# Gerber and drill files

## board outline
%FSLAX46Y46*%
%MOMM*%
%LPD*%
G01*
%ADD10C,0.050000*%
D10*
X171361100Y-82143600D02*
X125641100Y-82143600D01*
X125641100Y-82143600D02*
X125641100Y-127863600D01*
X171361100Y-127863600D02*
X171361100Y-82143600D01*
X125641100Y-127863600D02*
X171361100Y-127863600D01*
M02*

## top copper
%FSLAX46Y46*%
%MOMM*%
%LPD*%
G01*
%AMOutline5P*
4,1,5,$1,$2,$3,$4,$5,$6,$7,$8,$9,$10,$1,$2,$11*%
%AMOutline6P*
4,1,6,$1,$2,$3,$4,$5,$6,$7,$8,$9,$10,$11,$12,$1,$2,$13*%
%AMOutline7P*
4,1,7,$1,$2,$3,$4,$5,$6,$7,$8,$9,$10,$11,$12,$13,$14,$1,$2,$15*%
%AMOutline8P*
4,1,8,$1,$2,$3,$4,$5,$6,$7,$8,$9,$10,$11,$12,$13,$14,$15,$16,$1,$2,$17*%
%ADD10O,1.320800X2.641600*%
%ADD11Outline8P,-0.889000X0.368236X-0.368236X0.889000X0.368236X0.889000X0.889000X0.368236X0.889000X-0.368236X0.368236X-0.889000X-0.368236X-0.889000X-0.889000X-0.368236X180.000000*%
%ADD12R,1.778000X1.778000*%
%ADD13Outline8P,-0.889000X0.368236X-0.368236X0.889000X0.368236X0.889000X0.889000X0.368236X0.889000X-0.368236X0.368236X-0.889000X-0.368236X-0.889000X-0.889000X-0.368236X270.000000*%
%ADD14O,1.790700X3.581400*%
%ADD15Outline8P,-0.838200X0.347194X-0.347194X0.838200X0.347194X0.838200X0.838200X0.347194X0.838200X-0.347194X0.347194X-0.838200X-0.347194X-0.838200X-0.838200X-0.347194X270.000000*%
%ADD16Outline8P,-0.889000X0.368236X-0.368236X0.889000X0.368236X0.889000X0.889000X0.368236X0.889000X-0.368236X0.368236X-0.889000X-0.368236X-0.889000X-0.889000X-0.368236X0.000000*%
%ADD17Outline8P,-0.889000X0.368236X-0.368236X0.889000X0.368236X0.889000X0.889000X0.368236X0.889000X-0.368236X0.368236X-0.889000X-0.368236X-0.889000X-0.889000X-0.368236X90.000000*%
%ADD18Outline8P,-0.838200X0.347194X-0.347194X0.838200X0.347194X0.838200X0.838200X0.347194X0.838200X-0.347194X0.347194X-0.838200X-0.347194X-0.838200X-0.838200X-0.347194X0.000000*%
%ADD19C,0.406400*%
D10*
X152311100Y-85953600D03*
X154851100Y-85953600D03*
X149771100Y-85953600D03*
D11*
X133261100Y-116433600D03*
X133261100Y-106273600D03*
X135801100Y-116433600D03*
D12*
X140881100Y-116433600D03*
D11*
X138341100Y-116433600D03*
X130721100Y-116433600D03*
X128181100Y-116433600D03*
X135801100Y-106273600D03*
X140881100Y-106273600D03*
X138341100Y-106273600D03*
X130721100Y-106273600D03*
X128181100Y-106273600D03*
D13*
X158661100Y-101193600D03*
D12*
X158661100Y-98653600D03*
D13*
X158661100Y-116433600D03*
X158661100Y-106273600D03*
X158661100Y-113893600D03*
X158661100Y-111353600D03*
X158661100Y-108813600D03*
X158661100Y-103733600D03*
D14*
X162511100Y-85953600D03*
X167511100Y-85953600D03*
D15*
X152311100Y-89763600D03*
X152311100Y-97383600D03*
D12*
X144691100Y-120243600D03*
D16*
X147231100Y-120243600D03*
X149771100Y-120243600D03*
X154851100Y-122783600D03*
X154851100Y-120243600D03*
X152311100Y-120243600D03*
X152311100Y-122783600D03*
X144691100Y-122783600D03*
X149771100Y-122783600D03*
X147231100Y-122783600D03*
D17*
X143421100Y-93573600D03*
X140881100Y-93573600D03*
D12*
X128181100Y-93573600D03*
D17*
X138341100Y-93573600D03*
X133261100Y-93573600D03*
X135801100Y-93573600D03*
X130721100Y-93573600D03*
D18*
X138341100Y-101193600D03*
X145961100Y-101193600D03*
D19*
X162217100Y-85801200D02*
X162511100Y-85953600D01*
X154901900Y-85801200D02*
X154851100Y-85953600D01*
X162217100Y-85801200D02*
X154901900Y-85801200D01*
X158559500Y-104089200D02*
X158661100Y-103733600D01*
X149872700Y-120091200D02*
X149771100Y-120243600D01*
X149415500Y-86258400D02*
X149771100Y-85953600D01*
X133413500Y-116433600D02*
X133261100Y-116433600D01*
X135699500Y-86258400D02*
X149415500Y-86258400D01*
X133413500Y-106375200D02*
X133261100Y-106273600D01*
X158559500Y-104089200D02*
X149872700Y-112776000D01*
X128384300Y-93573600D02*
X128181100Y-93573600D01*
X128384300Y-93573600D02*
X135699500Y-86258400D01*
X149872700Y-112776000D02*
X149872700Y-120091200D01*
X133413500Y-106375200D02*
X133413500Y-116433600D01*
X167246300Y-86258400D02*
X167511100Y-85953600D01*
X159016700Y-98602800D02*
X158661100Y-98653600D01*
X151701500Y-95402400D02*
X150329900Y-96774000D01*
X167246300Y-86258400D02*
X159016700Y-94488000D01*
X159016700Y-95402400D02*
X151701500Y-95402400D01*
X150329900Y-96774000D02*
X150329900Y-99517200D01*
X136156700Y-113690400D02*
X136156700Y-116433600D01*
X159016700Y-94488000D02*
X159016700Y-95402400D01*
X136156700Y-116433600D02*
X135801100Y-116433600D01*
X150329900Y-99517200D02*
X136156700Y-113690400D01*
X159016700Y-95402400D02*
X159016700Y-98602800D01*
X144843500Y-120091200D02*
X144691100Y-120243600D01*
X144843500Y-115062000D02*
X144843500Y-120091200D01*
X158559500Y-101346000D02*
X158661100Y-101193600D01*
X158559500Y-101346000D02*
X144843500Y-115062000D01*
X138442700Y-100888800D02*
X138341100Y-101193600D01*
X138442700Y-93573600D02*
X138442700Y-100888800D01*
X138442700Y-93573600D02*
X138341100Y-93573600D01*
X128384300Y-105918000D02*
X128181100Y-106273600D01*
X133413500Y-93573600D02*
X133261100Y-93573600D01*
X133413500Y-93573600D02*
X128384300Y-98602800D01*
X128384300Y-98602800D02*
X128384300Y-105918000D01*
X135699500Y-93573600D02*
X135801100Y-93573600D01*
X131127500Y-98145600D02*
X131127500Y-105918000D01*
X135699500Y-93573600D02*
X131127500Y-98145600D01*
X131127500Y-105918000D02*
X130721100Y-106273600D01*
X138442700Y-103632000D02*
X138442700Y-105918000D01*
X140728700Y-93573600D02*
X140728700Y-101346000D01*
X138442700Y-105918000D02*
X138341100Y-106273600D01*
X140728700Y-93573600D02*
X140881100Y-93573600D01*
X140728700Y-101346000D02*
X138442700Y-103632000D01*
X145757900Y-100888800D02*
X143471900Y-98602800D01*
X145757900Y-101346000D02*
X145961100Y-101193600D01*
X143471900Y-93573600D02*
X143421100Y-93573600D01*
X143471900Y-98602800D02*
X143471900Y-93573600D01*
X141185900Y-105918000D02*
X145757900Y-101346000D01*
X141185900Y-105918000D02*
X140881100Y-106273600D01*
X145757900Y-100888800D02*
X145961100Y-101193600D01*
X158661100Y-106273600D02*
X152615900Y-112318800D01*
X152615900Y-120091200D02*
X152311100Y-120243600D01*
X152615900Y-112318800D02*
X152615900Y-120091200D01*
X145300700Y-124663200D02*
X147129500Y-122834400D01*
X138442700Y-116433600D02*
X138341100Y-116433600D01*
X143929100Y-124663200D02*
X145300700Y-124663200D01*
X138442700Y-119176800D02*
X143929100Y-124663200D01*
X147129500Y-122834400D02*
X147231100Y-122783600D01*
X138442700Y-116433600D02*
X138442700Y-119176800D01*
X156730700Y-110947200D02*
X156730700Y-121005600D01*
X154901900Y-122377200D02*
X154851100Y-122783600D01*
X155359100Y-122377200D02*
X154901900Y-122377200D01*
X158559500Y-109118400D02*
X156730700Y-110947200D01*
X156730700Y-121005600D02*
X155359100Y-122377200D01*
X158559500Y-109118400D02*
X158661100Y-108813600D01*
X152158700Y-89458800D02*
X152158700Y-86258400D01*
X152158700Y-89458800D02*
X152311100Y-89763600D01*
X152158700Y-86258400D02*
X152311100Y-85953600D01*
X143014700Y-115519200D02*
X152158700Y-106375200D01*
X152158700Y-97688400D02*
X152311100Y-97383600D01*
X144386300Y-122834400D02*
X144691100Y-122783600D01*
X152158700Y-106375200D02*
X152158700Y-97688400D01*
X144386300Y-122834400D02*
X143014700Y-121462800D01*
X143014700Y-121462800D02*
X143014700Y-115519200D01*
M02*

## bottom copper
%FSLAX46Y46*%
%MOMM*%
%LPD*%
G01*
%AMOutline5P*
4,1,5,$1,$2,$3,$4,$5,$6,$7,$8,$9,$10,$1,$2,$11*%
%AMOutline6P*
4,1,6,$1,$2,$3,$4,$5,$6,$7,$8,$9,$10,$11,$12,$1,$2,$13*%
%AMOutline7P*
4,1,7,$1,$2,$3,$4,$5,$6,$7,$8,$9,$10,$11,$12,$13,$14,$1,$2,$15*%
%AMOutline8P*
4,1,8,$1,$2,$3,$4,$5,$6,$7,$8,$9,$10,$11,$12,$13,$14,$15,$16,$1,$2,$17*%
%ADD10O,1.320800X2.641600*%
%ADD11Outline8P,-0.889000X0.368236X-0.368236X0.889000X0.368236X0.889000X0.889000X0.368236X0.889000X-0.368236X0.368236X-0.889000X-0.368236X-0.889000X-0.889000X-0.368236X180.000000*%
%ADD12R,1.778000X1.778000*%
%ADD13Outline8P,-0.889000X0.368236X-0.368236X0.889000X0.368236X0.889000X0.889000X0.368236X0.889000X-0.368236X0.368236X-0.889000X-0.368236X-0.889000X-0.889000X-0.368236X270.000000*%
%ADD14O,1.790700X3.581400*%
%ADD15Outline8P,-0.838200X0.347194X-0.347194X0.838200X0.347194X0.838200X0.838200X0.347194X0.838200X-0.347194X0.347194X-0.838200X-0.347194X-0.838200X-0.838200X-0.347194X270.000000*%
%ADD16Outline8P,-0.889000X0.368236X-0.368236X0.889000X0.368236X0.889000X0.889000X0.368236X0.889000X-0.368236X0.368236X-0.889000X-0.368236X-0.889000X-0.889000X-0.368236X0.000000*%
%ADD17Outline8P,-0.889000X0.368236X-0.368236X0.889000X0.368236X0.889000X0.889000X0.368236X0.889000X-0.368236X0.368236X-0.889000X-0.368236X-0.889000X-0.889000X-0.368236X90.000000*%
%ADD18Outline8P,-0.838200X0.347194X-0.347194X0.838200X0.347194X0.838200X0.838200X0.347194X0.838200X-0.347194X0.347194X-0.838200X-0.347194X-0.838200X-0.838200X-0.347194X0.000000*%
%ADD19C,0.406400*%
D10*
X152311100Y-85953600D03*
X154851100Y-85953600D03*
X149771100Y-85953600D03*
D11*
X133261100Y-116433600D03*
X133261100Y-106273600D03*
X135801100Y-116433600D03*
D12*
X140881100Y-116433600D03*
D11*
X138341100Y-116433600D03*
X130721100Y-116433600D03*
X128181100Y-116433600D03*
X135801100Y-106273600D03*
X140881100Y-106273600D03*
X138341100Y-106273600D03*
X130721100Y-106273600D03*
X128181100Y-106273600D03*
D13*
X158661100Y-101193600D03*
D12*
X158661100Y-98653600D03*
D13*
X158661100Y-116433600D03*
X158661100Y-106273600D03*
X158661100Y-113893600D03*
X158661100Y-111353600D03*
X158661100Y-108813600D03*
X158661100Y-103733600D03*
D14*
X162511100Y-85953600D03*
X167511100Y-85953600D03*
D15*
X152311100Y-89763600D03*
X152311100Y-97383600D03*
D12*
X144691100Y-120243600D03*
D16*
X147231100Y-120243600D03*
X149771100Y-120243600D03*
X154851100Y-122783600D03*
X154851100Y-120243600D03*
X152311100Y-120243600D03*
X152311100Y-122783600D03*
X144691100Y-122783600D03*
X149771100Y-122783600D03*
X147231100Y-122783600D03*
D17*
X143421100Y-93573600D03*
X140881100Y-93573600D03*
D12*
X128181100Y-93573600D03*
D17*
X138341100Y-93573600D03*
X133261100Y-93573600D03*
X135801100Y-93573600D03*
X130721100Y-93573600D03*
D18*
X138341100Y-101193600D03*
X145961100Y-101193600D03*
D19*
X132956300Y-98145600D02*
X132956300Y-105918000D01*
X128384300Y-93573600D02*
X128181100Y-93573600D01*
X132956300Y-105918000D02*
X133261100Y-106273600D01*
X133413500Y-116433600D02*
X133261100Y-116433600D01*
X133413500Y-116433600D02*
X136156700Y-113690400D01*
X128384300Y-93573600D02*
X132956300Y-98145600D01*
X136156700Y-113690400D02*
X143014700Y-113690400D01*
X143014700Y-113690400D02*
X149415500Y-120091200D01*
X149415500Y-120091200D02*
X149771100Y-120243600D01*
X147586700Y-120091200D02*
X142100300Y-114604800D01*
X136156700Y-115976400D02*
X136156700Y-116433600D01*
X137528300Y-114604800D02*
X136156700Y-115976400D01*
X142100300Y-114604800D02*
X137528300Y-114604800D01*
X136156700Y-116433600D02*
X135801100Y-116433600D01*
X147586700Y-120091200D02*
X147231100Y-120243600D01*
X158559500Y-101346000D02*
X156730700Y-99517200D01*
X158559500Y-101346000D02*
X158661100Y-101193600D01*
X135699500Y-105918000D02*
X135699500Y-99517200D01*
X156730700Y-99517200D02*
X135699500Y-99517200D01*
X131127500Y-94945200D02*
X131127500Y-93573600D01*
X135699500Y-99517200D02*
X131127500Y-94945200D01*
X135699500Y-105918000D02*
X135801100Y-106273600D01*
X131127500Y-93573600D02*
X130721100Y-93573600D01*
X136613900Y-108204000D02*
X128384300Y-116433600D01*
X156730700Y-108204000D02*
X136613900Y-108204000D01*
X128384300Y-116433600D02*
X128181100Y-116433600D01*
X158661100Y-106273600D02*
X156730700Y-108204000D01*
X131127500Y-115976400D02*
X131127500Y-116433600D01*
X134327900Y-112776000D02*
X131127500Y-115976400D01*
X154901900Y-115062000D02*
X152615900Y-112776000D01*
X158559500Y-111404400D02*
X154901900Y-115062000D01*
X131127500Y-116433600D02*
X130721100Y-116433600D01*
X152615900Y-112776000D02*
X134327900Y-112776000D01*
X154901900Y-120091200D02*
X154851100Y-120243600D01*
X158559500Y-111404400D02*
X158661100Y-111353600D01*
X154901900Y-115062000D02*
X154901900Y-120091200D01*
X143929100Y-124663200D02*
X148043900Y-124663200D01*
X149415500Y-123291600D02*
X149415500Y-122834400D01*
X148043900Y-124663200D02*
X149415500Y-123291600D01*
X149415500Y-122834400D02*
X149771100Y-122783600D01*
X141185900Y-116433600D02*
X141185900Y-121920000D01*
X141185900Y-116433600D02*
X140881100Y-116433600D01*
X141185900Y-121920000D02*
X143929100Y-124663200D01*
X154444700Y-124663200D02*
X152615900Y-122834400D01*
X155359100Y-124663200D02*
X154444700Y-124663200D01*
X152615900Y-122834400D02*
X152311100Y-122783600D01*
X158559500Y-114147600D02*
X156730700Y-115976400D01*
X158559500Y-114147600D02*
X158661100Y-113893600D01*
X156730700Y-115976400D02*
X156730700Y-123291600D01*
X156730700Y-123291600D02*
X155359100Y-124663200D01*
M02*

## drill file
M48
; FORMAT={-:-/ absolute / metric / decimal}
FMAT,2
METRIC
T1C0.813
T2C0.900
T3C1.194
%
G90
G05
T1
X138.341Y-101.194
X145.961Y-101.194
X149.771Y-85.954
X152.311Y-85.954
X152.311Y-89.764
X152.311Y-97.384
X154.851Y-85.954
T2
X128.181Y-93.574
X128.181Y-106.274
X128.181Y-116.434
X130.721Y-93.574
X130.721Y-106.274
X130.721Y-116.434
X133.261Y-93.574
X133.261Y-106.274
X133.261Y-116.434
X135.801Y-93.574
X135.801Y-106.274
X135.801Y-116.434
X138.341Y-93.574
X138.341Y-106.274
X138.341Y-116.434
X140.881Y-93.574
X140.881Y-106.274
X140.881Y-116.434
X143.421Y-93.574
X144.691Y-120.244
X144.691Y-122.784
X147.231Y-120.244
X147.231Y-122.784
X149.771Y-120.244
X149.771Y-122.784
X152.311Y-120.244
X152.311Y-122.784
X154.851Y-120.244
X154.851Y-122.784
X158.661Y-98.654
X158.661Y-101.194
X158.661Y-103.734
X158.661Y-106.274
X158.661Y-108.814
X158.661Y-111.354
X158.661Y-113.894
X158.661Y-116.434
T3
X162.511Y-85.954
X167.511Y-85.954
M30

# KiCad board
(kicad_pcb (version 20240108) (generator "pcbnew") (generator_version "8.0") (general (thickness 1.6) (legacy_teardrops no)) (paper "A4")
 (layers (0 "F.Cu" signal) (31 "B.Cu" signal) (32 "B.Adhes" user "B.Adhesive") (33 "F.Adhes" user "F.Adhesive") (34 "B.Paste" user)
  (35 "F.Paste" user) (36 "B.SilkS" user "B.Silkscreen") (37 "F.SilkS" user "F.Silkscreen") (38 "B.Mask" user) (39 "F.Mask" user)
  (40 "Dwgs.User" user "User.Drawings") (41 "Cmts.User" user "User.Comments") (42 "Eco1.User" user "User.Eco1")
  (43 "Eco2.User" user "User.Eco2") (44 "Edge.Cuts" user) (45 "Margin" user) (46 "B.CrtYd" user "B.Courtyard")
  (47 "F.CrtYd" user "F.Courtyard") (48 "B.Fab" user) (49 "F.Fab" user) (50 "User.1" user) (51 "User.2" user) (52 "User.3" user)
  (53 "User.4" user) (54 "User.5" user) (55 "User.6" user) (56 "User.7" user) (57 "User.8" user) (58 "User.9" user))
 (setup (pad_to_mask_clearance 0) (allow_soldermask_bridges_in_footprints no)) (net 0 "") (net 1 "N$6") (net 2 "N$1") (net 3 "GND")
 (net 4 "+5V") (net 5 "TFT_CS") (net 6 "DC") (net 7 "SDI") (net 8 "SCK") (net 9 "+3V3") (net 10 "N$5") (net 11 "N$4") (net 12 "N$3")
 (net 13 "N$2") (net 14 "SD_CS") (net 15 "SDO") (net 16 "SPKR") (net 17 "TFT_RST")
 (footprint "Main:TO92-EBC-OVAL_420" (layer "F.Cu") (at 152.3111 84.6836)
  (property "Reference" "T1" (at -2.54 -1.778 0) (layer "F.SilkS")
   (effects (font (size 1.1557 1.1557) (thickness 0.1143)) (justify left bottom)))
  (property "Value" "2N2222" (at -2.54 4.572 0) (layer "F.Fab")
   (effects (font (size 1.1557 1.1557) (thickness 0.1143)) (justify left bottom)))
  (pad "B" thru_hole oval (at 0 1.27 90) (size 2.6416 1.3208) (drill 0.8128) (layers "*.Cu" "*.Mask") (remove_unused_layers no)
   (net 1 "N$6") (solder_mask_margin 0.1016) (thermal_bridge_angle 0))
  (pad "C" thru_hole oval (at 2.54 1.27 90) (size 2.6416 1.3208) (drill 0.8128) (layers "*.Cu" "*.Mask") (remove_unused_layers no)
   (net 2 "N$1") (solder_mask_margin 0.1016) (thermal_bridge_angle 0))
  (pad "E" thru_hole oval (at -2.54 1.27 90) (size 2.6416 1.3208) (drill 0.8128) (layers "*.Cu" "*.Mask") (remove_unused_layers no)
   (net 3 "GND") (solder_mask_margin 0.1016) (thermal_bridge_angle 0)))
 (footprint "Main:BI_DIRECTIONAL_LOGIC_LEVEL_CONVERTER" (layer "F.Cu") (at 134.5311 111.3536 180)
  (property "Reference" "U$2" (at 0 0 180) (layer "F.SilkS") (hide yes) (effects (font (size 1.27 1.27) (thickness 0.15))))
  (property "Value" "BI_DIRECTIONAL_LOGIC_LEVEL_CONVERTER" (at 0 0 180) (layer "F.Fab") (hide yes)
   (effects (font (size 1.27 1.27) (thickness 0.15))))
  (pad "GND1" thru_hole roundrect (at 1.27 -5.08 180) (size 1.778 1.778) (drill 0.9) (layers "*.Cu" "*.Mask") (remove_unused_layers no)
   (roundrect_rratio 0.25) (chamfer_ratio 0.2928932188) (chamfer top_left top_right bottom_left bottom_right) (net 3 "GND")
   (solder_mask_margin 0.1016) (thermal_bridge_angle 0))
  (pad "GND2" thru_hole roundrect (at 1.27 5.08 180) (size 1.778 1.778) (drill 0.9) (layers "*.Cu" "*.Mask") (remove_unused_layers no)
   (roundrect_rratio 0.25) (chamfer_ratio 0.2928932188) (chamfer top_left top_right bottom_left bottom_right) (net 3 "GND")
   (solder_mask_margin 0.1016) (thermal_bridge_angle 0))
  (pad "HV" thru_hole roundrect (at -1.27 -5.08 180) (size 1.778 1.778) (drill 0.9) (layers "*.Cu" "*.Mask") (remove_unused_layers no)
   (roundrect_rratio 0.25) (chamfer_ratio 0.2928932188) (chamfer top_left top_right bottom_left bottom_right) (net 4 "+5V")
   (solder_mask_margin 0.1016) (thermal_bridge_angle 0))
  (pad "HV1" thru_hole rect (at -6.35 -5.08 180) (size 1.778 1.778) (drill 0.9) (layers "*.Cu" "*.Mask") (remove_unused_layers no)
   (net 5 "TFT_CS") (solder_mask_margin 0.1016) (thermal_bridge_angle 0))
  (pad "HV2" thru_hole roundrect (at -3.81 -5.08 180) (size 1.778 1.778) (drill 0.9) (layers "*.Cu" "*.Mask") (remove_unused_layers no)
   (roundrect_rratio 0.25) (chamfer_ratio 0.2928932188) (chamfer top_left top_right bottom_left bottom_right) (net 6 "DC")
   (solder_mask_margin 0.1016) (thermal_bridge_angle 0))
  (pad "HV3" thru_hole roundrect (at 3.81 -5.08 180) (size 1.778 1.778) (drill 0.9) (layers "*.Cu" "*.Mask") (remove_unused_layers no)
   (roundrect_rratio 0.25) (chamfer_ratio 0.2928932188) (chamfer top_left top_right bottom_left bottom_right) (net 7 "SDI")
   (solder_mask_margin 0.1016) (thermal_bridge_angle 0))
  (pad "HV4" thru_hole roundrect (at 6.35 -5.08 180) (size 1.778 1.778) (drill 0.9) (layers "*.Cu" "*.Mask") (remove_unused_layers no)
   (roundrect_rratio 0.25) (chamfer_ratio 0.2928932188) (chamfer top_left top_right bottom_left bottom_right) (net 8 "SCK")
   (solder_mask_margin 0.1016) (thermal_bridge_angle 0))
  (pad "LV" thru_hole roundrect (at -1.27 5.08 180) (size 1.778 1.778) (drill 0.9) (layers "*.Cu" "*.Mask") (remove_unused_layers no)
   (roundrect_rratio 0.25) (chamfer_ratio 0.2928932188) (chamfer top_left top_right bottom_left bottom_right) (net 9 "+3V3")
   (solder_mask_margin 0.1016) (thermal_bridge_angle 0))
  (pad "LV1" thru_hole roundrect (at -6.35 5.08 180) (size 1.778 1.778) (drill 0.9) (layers "*.Cu" "*.Mask") (remove_unused_layers no)
   (roundrect_rratio 0.25) (chamfer_ratio 0.2928932188) (chamfer top_left top_right bottom_left bottom_right) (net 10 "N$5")
   (solder_mask_margin 0.1016) (thermal_bridge_angle 0))
  (pad "LV2" thru_hole roundrect (at -3.81 5.08 180) (size 1.778 1.778) (drill 0.9) (layers "*.Cu" "*.Mask") (remove_unused_layers no)
   (roundrect_rratio 0.25) (chamfer_ratio 0.2928932188) (chamfer top_left top_right bottom_left bottom_right) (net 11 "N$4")
   (solder_mask_margin 0.1016) (thermal_bridge_angle 0))
  (pad "LV3" thru_hole roundrect (at 3.81 5.08 180) (size 1.778 1.778) (drill 0.9) (layers "*.Cu" "*.Mask") (remove_unused_layers no)
   (roundrect_rratio 0.25) (chamfer_ratio 0.2928932188) (chamfer top_left top_right bottom_left bottom_right) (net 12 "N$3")
   (solder_mask_margin 0.1016) (thermal_bridge_angle 0))
  (pad "LV4" thru_hole roundrect (at 6.35 5.08 180) (size 1.778 1.778) (drill 0.9) (layers "*.Cu" "*.Mask") (remove_unused_layers no)
   (roundrect_rratio 0.25) (chamfer_ratio 0.2928932188) (chamfer top_left top_right bottom_left bottom_right) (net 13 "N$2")
   (solder_mask_margin 0.1016) (thermal_bridge_angle 0)))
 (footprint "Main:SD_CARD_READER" (layer "F.Cu") (at 158.6611 107.5436 -90)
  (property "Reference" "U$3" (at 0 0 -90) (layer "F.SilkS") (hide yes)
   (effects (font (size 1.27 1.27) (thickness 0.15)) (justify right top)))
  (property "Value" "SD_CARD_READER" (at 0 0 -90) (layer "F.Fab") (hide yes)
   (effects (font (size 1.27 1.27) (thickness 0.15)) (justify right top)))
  (pad "3V" thru_hole roundrect (at -6.35 0 270) (size 1.778 1.778) (drill 0.9) (layers "*.Cu" "*.Mask") (remove_unused_layers no)
   (roundrect_rratio 0.25) (chamfer_ratio 0.2928932188) (chamfer top_left top_right bottom_left bottom_right) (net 9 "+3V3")
   (solder_mask_margin 0.1016) (thermal_bridge_angle 0))
  (pad "5V" thru_hole rect (at -8.89 0 270) (size 1.778 1.778) (drill 0.9) (layers "*.Cu" "*.Mask") (remove_unused_layers no) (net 4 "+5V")
   (solder_mask_margin 0.1016) (thermal_bridge_angle 0))
  (pad "CD" thru_hole roundrect (at 8.89 0 270) (size 1.778 1.778) (drill 0.9) (layers "*.Cu" "*.Mask") (remove_unused_layers no)
   (roundrect_rratio 0.25) (chamfer_ratio 0.2928932188) (chamfer top_left top_right bottom_left bottom_right) (solder_mask_margin 0.1016)
   (thermal_bridge_angle 0))
  (pad "CLK" thru_hole roundrect (at -1.27 0 270) (size 1.778 1.778) (drill 0.9) (layers "*.Cu" "*.Mask") (remove_unused_layers no)
   (roundrect_rratio 0.25) (chamfer_ratio 0.2928932188) (chamfer top_left top_right bottom_left bottom_right) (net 8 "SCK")
   (solder_mask_margin 0.1016) (thermal_bridge_angle 0))
  (pad "CS" thru_hole roundrect (at 6.35 0 270) (size 1.778 1.778) (drill 0.9) (layers "*.Cu" "*.Mask") (remove_unused_layers no)
   (roundrect_rratio 0.25) (chamfer_ratio 0.2928932188) (chamfer top_left top_right bottom_left bottom_right) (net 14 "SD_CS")
   (solder_mask_margin 0.1016) (thermal_bridge_angle 0))
  (pad "DI" thru_hole roundrect (at 3.81 0 270) (size 1.778 1.778) (drill 0.9) (layers "*.Cu" "*.Mask") (remove_unused_layers no)
   (roundrect_rratio 0.25) (chamfer_ratio 0.2928932188) (chamfer top_left top_right bottom_left bottom_right) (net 7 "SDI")
   (solder_mask_margin 0.1016) (thermal_bridge_angle 0))
  (pad "DO" thru_hole roundrect (at 1.27 0 270) (size 1.778 1.778) (drill 0.9) (layers "*.Cu" "*.Mask") (remove_unused_layers no)
   (roundrect_rratio 0.25) (chamfer_ratio 0.2928932188) (chamfer top_left top_right bottom_left bottom_right) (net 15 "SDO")
   (solder_mask_margin 0.1016) (thermal_bridge_angle 0))
  (pad "GND" thru_hole roundrect (at -3.81 0 270) (size 1.778 1.778) (drill 0.9) (layers "*.Cu" "*.Mask") (remove_unused_layers no)
   (roundrect_rratio 0.25) (chamfer_ratio 0.2928932188) (chamfer top_left top_right bottom_left bottom_right) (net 3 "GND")
   (solder_mask_margin 0.1016) (thermal_bridge_angle 0)))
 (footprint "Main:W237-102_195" (layer "F.Cu") (at 165.0111 84.6836)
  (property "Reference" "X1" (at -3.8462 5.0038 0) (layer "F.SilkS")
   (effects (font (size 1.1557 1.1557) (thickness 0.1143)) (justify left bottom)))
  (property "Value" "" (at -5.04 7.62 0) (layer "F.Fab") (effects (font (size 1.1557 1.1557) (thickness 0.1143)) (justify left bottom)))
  (pad "1" thru_hole oval (at -2.5 1.27 90) (size 3.5814 1.7907) (drill 1.1938) (layers "*.Cu" "*.Mask") (remove_unused_layers no)
   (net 2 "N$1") (solder_mask_margin 0.1016) (thermal_bridge_angle 0))
  (pad "2" thru_hole oval (at 2.5 1.27 90) (size 3.5814 1.7907) (drill 1.1938) (layers "*.Cu" "*.Mask") (remove_unused_layers no)
   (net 4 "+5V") (solder_mask_margin 0.1016) (thermal_bridge_angle 0)))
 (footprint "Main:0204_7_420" (layer "F.Cu") (at 152.3111 93.5736 -90)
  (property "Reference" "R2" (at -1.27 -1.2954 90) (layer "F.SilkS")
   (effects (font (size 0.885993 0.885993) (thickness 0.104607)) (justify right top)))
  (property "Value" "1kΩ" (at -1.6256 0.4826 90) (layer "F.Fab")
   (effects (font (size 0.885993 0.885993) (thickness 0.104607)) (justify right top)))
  (pad "1" thru_hole roundrect (at -3.81 0 270) (size 1.6764 1.6764) (drill 0.8128) (layers "*.Cu" "*.Mask") (remove_unused_layers no)
   (roundrect_rratio 0.25) (chamfer_ratio 0.2928932188) (chamfer top_left top_right bottom_left bottom_right) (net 1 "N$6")
   (solder_mask_margin 0.1016) (thermal_bridge_angle 0))
  (pad "2" thru_hole roundrect (at 3.81 0 270) (size 1.6764 1.6764) (drill 0.8128) (layers "*.Cu" "*.Mask") (remove_unused_layers no)
   (roundrect_rratio 0.25) (chamfer_ratio 0.2928932188) (chamfer top_left top_right bottom_left bottom_right) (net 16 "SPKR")
   (solder_mask_margin 0.1016) (thermal_bridge_angle 0)))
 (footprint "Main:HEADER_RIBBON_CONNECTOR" (layer "F.Cu") (at 149.7711 121.5136)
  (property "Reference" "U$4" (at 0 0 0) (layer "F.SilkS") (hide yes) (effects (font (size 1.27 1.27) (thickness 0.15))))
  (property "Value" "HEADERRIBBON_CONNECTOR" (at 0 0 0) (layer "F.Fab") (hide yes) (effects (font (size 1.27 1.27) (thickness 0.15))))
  (pad "3V3" thru_hole rect (at -5.08 -1.27) (size 1.778 1.778) (drill 0.9) (layers "*.Cu" "*.Mask") (remove_unused_layers no)
   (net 9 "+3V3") (solder_mask_margin 0.1016) (thermal_bridge_angle 0))
  (pad "5V" thru_hole roundrect (at -2.54 -1.27) (size 1.778 1.778) (drill 0.9) (layers "*.Cu" "*.Mask") (remove_unused_layers no)
   (roundrect_rratio 0.25) (chamfer_ratio 0.2928932188) (chamfer top_left top_right bottom_left bottom_right) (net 4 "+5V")
   (solder_mask_margin 0.1016) (thermal_bridge_angle 0))
  (pad "GND" thru_hole roundrect (at 0 -1.27) (size 1.778 1.778) (drill 0.9) (layers "*.Cu" "*.Mask") (remove_unused_layers no)
   (roundrect_rratio 0.25) (chamfer_ratio 0.2928932188) (chamfer top_left top_right bottom_left bottom_right) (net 3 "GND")
   (solder_mask_margin 0.1016) (thermal_bridge_angle 0))
  (pad "MISO" thru_hole roundrect (at 5.08 1.27) (size 1.778 1.778) (drill 0.9) (layers "*.Cu" "*.Mask") (remove_unused_layers no)
   (roundrect_rratio 0.25) (chamfer_ratio 0.2928932188) (chamfer top_left top_right bottom_left bottom_right) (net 15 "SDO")
   (solder_mask_margin 0.1016) (thermal_bridge_angle 0))
  (pad "MOSI" thru_hole roundrect (at 5.08 -1.27) (size 1.778 1.778) (drill 0.9) (layers "*.Cu" "*.Mask") (remove_unused_layers no)
   (roundrect_rratio 0.25) (chamfer_ratio 0.2928932188) (chamfer top_left top_right bottom_left bottom_right) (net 7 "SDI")
   (solder_mask_margin 0.1016) (thermal_bridge_angle 0))
  (pad "SCK" thru_hole roundrect (at 2.54 -1.27) (size 1.778 1.778) (drill 0.9) (layers "*.Cu" "*.Mask") (remove_unused_layers no)
   (roundrect_rratio 0.25) (chamfer_ratio 0.2928932188) (chamfer top_left top_right bottom_left bottom_right) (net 8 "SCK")
   (solder_mask_margin 0.1016) (thermal_bridge_angle 0))
  (pad "SD_CS" thru_hole roundrect (at 2.54 1.27) (size 1.778 1.778) (drill 0.9) (layers "*.Cu" "*.Mask") (remove_unused_layers no)
   (roundrect_rratio 0.25) (chamfer_ratio 0.2928932188) (chamfer top_left top_right bottom_left bottom_right) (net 14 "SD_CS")
   (solder_mask_margin 0.1016) (thermal_bridge_angle 0))
  (pad "SPKR" thru_hole roundrect (at -5.08 1.27) (size 1.778 1.778) (drill 0.9) (layers "*.Cu" "*.Mask") (remove_unused_layers no)
   (roundrect_rratio 0.25) (chamfer_ratio 0.2928932188) (chamfer top_left top_right bottom_left bottom_right) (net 16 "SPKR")
   (solder_mask_margin 0.1016) (thermal_bridge_angle 0))
  (pad "TFT_CS" thru_hole roundrect (at 0 1.27) (size 1.778 1.778) (drill 0.9) (layers "*.Cu" "*.Mask") (remove_unused_layers no)
   (roundrect_rratio 0.25) (chamfer_ratio 0.2928932188) (chamfer top_left top_right bottom_left bottom_right) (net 5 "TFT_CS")
   (solder_mask_margin 0.1016) (thermal_bridge_angle 0))
  (pad "TFT_DC" thru_hole roundrect (at -2.54 1.27) (size 1.778 1.778) (drill 0.9) (layers "*.Cu" "*.Mask") (remove_unused_layers no)
   (roundrect_rratio 0.25) (chamfer_ratio 0.2928932188) (chamfer top_left top_right bottom_left bottom_right) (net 6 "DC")
   (solder_mask_margin 0.1016) (thermal_bridge_angle 0)))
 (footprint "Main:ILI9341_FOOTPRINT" (layer "F.Cu") (at 135.8011 78.3336 90)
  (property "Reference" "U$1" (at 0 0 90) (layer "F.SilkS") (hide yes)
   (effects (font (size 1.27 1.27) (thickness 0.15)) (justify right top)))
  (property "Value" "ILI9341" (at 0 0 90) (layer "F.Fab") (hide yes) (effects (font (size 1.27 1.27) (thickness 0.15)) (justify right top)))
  (pad "CS" thru_hole roundrect (at -15.24 7.62 90) (size 1.778 1.778) (drill 0.9) (layers "*.Cu" "*.Mask") (remove_unused_layers no)
   (roundrect_rratio 0.25) (chamfer_ratio 0.2928932188) (chamfer top_left top_right bottom_left bottom_right) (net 10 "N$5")
   (solder_mask_margin 0.1016) (thermal_bridge_angle 0))
  (pad "DC" thru_hole roundrect (at -15.24 5.08 90) (size 1.778 1.778) (drill 0.9) (layers "*.Cu" "*.Mask") (remove_unused_layers no)
   (roundrect_rratio 0.25) (chamfer_ratio 0.2928932188) (chamfer top_left top_right bottom_left bottom_right) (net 11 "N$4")
   (solder_mask_margin 0.1016) (thermal_bridge_angle 0))
  (pad "GND" thru_hole rect (at -15.24 -7.62 90) (size 1.778 1.778) (drill 0.9) (layers "*.Cu" "*.Mask") (remove_unused_layers no)
   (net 3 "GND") (solder_mask_margin 0.1016) (thermal_bridge_angle 0))
  (pad "RST" thru_hole roundrect (at -15.24 2.54 90) (size 1.778 1.778) (drill 0.9) (layers "*.Cu" "*.Mask") (remove_unused_layers no)
   (roundrect_rratio 0.25) (chamfer_ratio 0.2928932188) (chamfer top_left top_right bottom_left bottom_right) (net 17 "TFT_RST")
   (solder_mask_margin 0.1016) (thermal_bridge_angle 0))
  (pad "SCK" thru_hole roundrect (at -15.24 -2.54 90) (size 1.778 1.778) (drill 0.9) (layers "*.Cu" "*.Mask") (remove_unused_layers no)
   (roundrect_rratio 0.25) (chamfer_ratio 0.2928932188) (chamfer top_left top_right bottom_left bottom_right) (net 13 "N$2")
   (solder_mask_margin 0.1016) (thermal_bridge_angle 0))
  (pad "SDA" thru_hole roundrect (at -15.24 0 90) (size 1.778 1.778) (drill 0.9) (layers "*.Cu" "*.Mask") (remove_unused_layers no)
   (roundrect_rratio 0.25) (chamfer_ratio 0.2928932188) (chamfer top_left top_right bottom_left bottom_right) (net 12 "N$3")
   (solder_mask_margin 0.1016) (thermal_bridge_angle 0))
  (pad "VCC" thru_hole roundrect (at -15.24 -5.08 90) (size 1.778 1.778) (drill 0.9) (layers "*.Cu" "*.Mask") (remove_unused_layers no)
   (roundrect_rratio 0.25) (chamfer_ratio 0.2928932188) (chamfer top_left top_right bottom_left bottom_right) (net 9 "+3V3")
   (solder_mask_margin 0.1016) (thermal_bridge_angle 0)))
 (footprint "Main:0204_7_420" (layer "F.Cu") (at 142.1511 101.1936)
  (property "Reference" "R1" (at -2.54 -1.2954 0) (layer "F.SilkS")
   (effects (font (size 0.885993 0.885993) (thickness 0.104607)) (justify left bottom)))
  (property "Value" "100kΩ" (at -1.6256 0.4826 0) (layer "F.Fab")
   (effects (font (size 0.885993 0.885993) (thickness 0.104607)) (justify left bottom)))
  (pad "1" thru_hole roundrect (at -3.81 0) (size 1.6764 1.6764) (drill 0.8128) (layers "*.Cu" "*.Mask") (remove_unused_layers no)
   (roundrect_rratio 0.25) (chamfer_ratio 0.2928932188) (chamfer top_left top_right bottom_left bottom_right) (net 17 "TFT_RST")
   (solder_mask_margin 0.1016) (thermal_bridge_angle 0))
  (pad "2" thru_hole roundrect (at 3.81 0) (size 1.6764 1.6764) (drill 0.8128) (layers "*.Cu" "*.Mask") (remove_unused_layers no)
   (roundrect_rratio 0.25) (chamfer_ratio 0.2928932188) (chamfer top_left top_right bottom_left bottom_right) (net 10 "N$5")
   (solder_mask_margin 0.1016) (thermal_bridge_angle 0)))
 (gr_line (start 171.3611 82.1436) (end 125.6411 82.1436) (stroke (width 0.05) (type solid)) (layer "Edge.Cuts"))
 (gr_line (start 125.6411 82.1436) (end 125.6411 127.8636) (stroke (width 0.05) (type solid)) (layer "Edge.Cuts"))
 (gr_line (start 171.3611 127.8636) (end 171.3611 82.1436) (stroke (width 0.05) (type solid)) (layer "Edge.Cuts"))
 (gr_line (start 125.6411 127.8636) (end 171.3611 127.8636) (stroke (width 0.05) (type solid)) (layer "Edge.Cuts"))
 (segment (start 162.2171 85.8012) (end 162.5111 85.9536) (width 0.4064) (layer "F.Cu") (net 2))
 (segment (start 154.9019 85.8012) (end 154.8511 85.9536) (width 0.4064) (layer "F.Cu") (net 2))
 (segment (start 162.2171 85.8012) (end 154.9019 85.8012) (width 0.4064) (layer "F.Cu") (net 2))
 (segment (start 158.5595 104.0892) (end 158.6611 103.7336) (width 0.4064) (layer "F.Cu") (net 3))
 (segment (start 149.8727 120.0912) (end 149.7711 120.2436) (width 0.4064) (layer "F.Cu") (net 3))
 (segment (start 149.4155 86.2584) (end 149.7711 85.9536) (width 0.4064) (layer "F.Cu") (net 3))
 (segment (start 133.4135 116.4336) (end 133.2611 116.4336) (width 0.4064) (layer "F.Cu") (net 3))
 (segment (start 135.6995 86.2584) (end 149.4155 86.2584) (width 0.4064) (layer "F.Cu") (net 3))
 (segment (start 133.4135 106.3752) (end 133.2611 106.2736) (width 0.4064) (layer "F.Cu") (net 3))
 (segment (start 158.5595 104.0892) (end 149.8727 112.776) (width 0.4064) (layer "F.Cu") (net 3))
 (segment (start 128.3843 93.5736) (end 128.1811 93.5736) (width 0.4064) (layer "F.Cu") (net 3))
 (segment (start 128.3843 93.5736) (end 135.6995 86.2584) (width 0.4064) (layer "F.Cu") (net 3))
 (segment (start 149.8727 112.776) (end 149.8727 120.0912) (width 0.4064) (layer "F.Cu") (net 3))
 (segment (start 133.4135 106.3752) (end 133.4135 116.4336) (width 0.4064) (layer "F.Cu") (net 3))
 (segment (start 132.9563 98.1456) (end 132.9563 105.918) (width 0.4064) (layer "B.Cu") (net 3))
 (segment (start 128.3843 93.5736) (end 128.1811 93.5736) (width 0.4064) (layer "B.Cu") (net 3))
 (segment (start 132.9563 105.918) (end 133.2611 106.2736) (width 0.4064) (layer "B.Cu") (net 3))
 (segment (start 133.4135 116.4336) (end 133.2611 116.4336) (width 0.4064) (layer "B.Cu") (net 3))
 (segment (start 133.4135 116.4336) (end 136.1567 113.6904) (width 0.4064) (layer "B.Cu") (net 3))
 (segment (start 128.3843 93.5736) (end 132.9563 98.1456) (width 0.4064) (layer "B.Cu") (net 3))
 (segment (start 136.1567 113.6904) (end 143.0147 113.6904) (width 0.4064) (layer "B.Cu") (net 3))
 (segment (start 143.0147 113.6904) (end 149.4155 120.0912) (width 0.4064) (layer "B.Cu") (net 3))
 (segment (start 149.4155 120.0912) (end 149.7711 120.2436) (width 0.4064) (layer "B.Cu") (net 3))
 (segment (start 167.2463 86.2584) (end 167.5111 85.9536) (width 0.4064) (layer "F.Cu") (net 4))
 (segment (start 159.0167 98.6028) (end 158.6611 98.6536) (width 0.4064) (layer "F.Cu") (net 4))
 (segment (start 151.7015 95.4024) (end 150.3299 96.774) (width 0.4064) (layer "F.Cu") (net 4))
 (segment (start 167.2463 86.2584) (end 159.0167 94.488) (width 0.4064) (layer "F.Cu") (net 4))
 (segment (start 159.0167 95.4024) (end 151.7015 95.4024) (width 0.4064) (layer "F.Cu") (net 4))
 (segment (start 150.3299 96.774) (end 150.3299 99.5172) (width 0.4064) (layer "F.Cu") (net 4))
 (segment (start 136.1567 113.6904) (end 136.1567 116.4336) (width 0.4064) (layer "F.Cu") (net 4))
 (segment (start 159.0167 94.488) (end 159.0167 95.4024) (width 0.4064) (layer "F.Cu") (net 4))
 (segment (start 136.1567 116.4336) (end 135.8011 116.4336) (width 0.4064) (layer "F.Cu") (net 4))
 (segment (start 150.3299 99.5172) (end 136.1567 113.6904) (width 0.4064) (layer "F.Cu") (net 4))
 (segment (start 159.0167 95.4024) (end 159.0167 98.6028) (width 0.4064) (layer "F.Cu") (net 4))
 (segment (start 147.5867 120.0912) (end 142.1003 114.6048) (width 0.4064) (layer "B.Cu") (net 4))
 (segment (start 136.1567 115.9764) (end 136.1567 116.4336) (width 0.4064) (layer "B.Cu") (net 4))
 (segment (start 137.5283 114.6048) (end 136.1567 115.9764) (width 0.4064) (layer "B.Cu") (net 4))
 (segment (start 142.1003 114.6048) (end 137.5283 114.6048) (width 0.4064) (layer "B.Cu") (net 4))
 (segment (start 136.1567 116.4336) (end 135.8011 116.4336) (width 0.4064) (layer "B.Cu") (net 4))
 (segment (start 147.5867 120.0912) (end 147.2311 120.2436) (width 0.4064) (layer "B.Cu") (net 4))
 (segment (start 144.8435 120.0912) (end 144.6911 120.2436) (width 0.4064) (layer "F.Cu") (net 9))
 (segment (start 144.8435 115.062) (end 144.8435 120.0912) (width 0.4064) (layer "F.Cu") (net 9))
 (segment (start 158.5595 101.346) (end 158.6611 101.1936) (width 0.4064) (layer "F.Cu") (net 9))
 (segment (start 158.5595 101.346) (end 144.8435 115.062) (width 0.4064) (layer "F.Cu") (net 9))
 (segment (start 158.5595 101.346) (end 156.7307 99.5172) (width 0.4064) (layer "B.Cu") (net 9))
 (segment (start 158.5595 101.346) (end 158.6611 101.1936) (width 0.4064) (layer "B.Cu") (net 9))
 (segment (start 135.6995 105.918) (end 135.6995 99.5172) (width 0.4064) (layer "B.Cu") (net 9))
 (segment (start 156.7307 99.5172) (end 135.6995 99.5172) (width 0.4064) (layer "B.Cu") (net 9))
 (segment (start 131.1275 94.9452) (end 131.1275 93.5736) (width 0.4064) (layer "B.Cu") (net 9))
 (segment (start 135.6995 99.5172) (end 131.1275 94.9452) (width 0.4064) (layer "B.Cu") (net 9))
 (segment (start 135.6995 105.918) (end 135.8011 106.2736) (width 0.4064) (layer "B.Cu") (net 9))
 (segment (start 131.1275 93.5736) (end 130.7211 93.5736) (width 0.4064) (layer "B.Cu") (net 9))
 (segment (start 138.4427 100.8888) (end 138.3411 101.1936) (width 0.4064) (layer "F.Cu") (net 17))
 (segment (start 138.4427 93.5736) (end 138.4427 100.8888) (width 0.4064) (layer "F.Cu") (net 17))
 (segment (start 138.4427 93.5736) (end 138.3411 93.5736) (width 0.4064) (layer "F.Cu") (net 17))
 (segment (start 128.3843 105.918) (end 128.1811 106.2736) (width 0.4064) (layer "F.Cu") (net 13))
 (segment (start 133.4135 93.5736) (end 133.2611 93.5736) (width 0.4064) (layer "F.Cu") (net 13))
 (segment (start 133.4135 93.5736) (end 128.3843 98.6028) (width 0.4064) (layer "F.Cu") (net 13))
 (segment (start 128.3843 98.6028) (end 128.3843 105.918) (width 0.4064) (layer "F.Cu") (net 13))
 (segment (start 135.6995 93.5736) (end 135.8011 93.5736) (width 0.4064) (layer "F.Cu") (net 12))
 (segment (start 131.1275 98.1456) (end 131.1275 105.918) (width 0.4064) (layer "F.Cu") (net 12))
 (segment (start 135.6995 93.5736) (end 131.1275 98.1456) (width 0.4064) (layer "F.Cu") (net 12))
 (segment (start 131.1275 105.918) (end 130.7211 106.2736) (width 0.4064) (layer "F.Cu") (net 12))
 (segment (start 138.4427 103.632) (end 138.4427 105.918) (width 0.4064) (layer "F.Cu") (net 11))
 (segment (start 140.7287 93.5736) (end 140.7287 101.346) (width 0.4064) (layer "F.Cu") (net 11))
 (segment (start 138.4427 105.918) (end 138.3411 106.2736) (width 0.4064) (layer "F.Cu") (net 11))
 (segment (start 140.7287 93.5736) (end 140.8811 93.5736) (width 0.4064) (layer "F.Cu") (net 11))
 (segment (start 140.7287 101.346) (end 138.4427 103.632) (width 0.4064) (layer "F.Cu") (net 11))
 (segment (start 145.7579 100.8888) (end 143.4719 98.6028) (width 0.4064) (layer "F.Cu") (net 10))
 (segment (start 145.7579 101.346) (end 145.9611 101.1936) (width 0.4064) (layer "F.Cu") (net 10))
 (segment (start 143.4719 93.5736) (end 143.4211 93.5736) (width 0.4064) (layer "F.Cu") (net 10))
 (segment (start 143.4719 98.6028) (end 143.4719 93.5736) (width 0.4064) (layer "F.Cu") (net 10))
 (segment (start 141.1859 105.918) (end 145.7579 101.346) (width 0.4064) (layer "F.Cu") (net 10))
 (segment (start 141.1859 105.918) (end 140.8811 106.2736) (width 0.4064) (layer "F.Cu") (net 10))
 (segment (start 145.7579 100.8888) (end 145.9611 101.1936) (width 0.4064) (layer "F.Cu") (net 10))
 (segment (start 158.6611 106.2736) (end 152.6159 112.3188) (width 0.4064) (layer "F.Cu") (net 8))
 (segment (start 152.6159 120.0912) (end 152.3111 120.2436) (width 0.4064) (layer "F.Cu") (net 8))
 (segment (start 152.6159 112.3188) (end 152.6159 120.0912) (width 0.4064) (layer "F.Cu") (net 8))
 (segment (start 136.6139 108.204) (end 128.3843 116.4336) (width 0.4064) (layer "B.Cu") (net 8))
 (segment (start 156.7307 108.204) (end 136.6139 108.204) (width 0.4064) (layer "B.Cu") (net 8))
 (segment (start 128.3843 116.4336) (end 128.1811 116.4336) (width 0.4064) (layer "B.Cu") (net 8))
 (segment (start 158.6611 106.2736) (end 156.7307 108.204) (width 0.4064) (layer "B.Cu") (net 8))
 (segment (start 131.1275 115.9764) (end 131.1275 116.4336) (width 0.4064) (layer "B.Cu") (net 7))
 (segment (start 134.3279 112.776) (end 131.1275 115.9764) (width 0.4064) (layer "B.Cu") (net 7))
 (segment (start 154.9019 115.062) (end 152.6159 112.776) (width 0.4064) (layer "B.Cu") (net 7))
 (segment (start 158.5595 111.4044) (end 154.9019 115.062) (width 0.4064) (layer "B.Cu") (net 7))
 (segment (start 131.1275 116.4336) (end 130.7211 116.4336) (width 0.4064) (layer "B.Cu") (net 7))
 (segment (start 152.6159 112.776) (end 134.3279 112.776) (width 0.4064) (layer "B.Cu") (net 7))
 (segment (start 154.9019 120.0912) (end 154.8511 120.2436) (width 0.4064) (layer "B.Cu") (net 7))
 (segment (start 158.5595 111.4044) (end 158.6611 111.3536) (width 0.4064) (layer "B.Cu") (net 7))
 (segment (start 154.9019 115.062) (end 154.9019 120.0912) (width 0.4064) (layer "B.Cu") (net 7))
 (segment (start 145.3007 124.6632) (end 147.1295 122.8344) (width 0.4064) (layer "F.Cu") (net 6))
 (segment (start 138.4427 116.4336) (end 138.3411 116.4336) (width 0.4064) (layer "F.Cu") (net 6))
 (segment (start 143.9291 124.6632) (end 145.3007 124.6632) (width 0.4064) (layer "F.Cu") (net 6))
 (segment (start 138.4427 119.1768) (end 143.9291 124.6632) (width 0.4064) (layer "F.Cu") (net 6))
 (segment (start 147.1295 122.8344) (end 147.2311 122.7836) (width 0.4064) (layer "F.Cu") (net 6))
 (segment (start 138.4427 116.4336) (end 138.4427 119.1768) (width 0.4064) (layer "F.Cu") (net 6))
 (segment (start 143.9291 124.6632) (end 148.0439 124.6632) (width 0.4064) (layer "B.Cu") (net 5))
 (segment (start 149.4155 123.2916) (end 149.4155 122.8344) (width 0.4064) (layer "B.Cu") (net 5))
 (segment (start 148.0439 124.6632) (end 149.4155 123.2916) (width 0.4064) (layer "B.Cu") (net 5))
 (segment (start 149.4155 122.8344) (end 149.7711 122.7836) (width 0.4064) (layer "B.Cu") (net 5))
 (segment (start 141.1859 116.4336) (end 141.1859 121.92) (width 0.4064) (layer "B.Cu") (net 5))
 (segment (start 141.1859 116.4336) (end 140.8811 116.4336) (width 0.4064) (layer "B.Cu") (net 5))
 (segment (start 141.1859 121.92) (end 143.9291 124.6632) (width 0.4064) (layer "B.Cu") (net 5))
 (segment (start 156.7307 110.9472) (end 156.7307 121.0056) (width 0.4064) (layer "F.Cu") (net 15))
 (segment (start 154.9019 122.3772) (end 154.8511 122.7836) (width 0.4064) (layer "F.Cu") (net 15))
 (segment (start 155.3591 122.3772) (end 154.9019 122.3772) (width 0.4064) (layer "F.Cu") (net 15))
 (segment (start 158.5595 109.1184) (end 156.7307 110.9472) (width 0.4064) (layer "F.Cu") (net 15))
 (segment (start 156.7307 121.0056) (end 155.3591 122.3772) (width 0.4064) (layer "F.Cu") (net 15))
 (segment (start 158.5595 109.1184) (end 158.6611 108.8136) (width 0.4064) (layer "F.Cu") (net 15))
 (segment (start 154.4447 124.6632) (end 152.6159 122.8344) (width 0.4064) (layer "B.Cu") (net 14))
 (segment (start 155.3591 124.6632) (end 154.4447 124.6632) (width 0.4064) (layer "B.Cu") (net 14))
 (segment (start 152.6159 122.8344) (end 152.3111 122.7836) (width 0.4064) (layer "B.Cu") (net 14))
 (segment (start 158.5595 114.1476) (end 156.7307 115.9764) (width 0.4064) (layer "B.Cu") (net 14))
 (segment (start 158.5595 114.1476) (end 158.6611 113.8936) (width 0.4064) (layer "B.Cu") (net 14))
 (segment (start 156.7307 115.9764) (end 156.7307 123.2916) (width 0.4064) (layer "B.Cu") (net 14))
 (segment (start 156.7307 123.2916) (end 155.3591 124.6632) (width 0.4064) (layer "B.Cu") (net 14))
 (segment (start 152.1587 89.4588) (end 152.1587 86.2584) (width 0.4064) (layer "F.Cu") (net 1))
 (segment (start 152.1587 89.4588) (end 152.3111 89.7636) (width 0.4064) (layer "F.Cu") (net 1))
 (segment (start 152.1587 86.2584) (end 152.3111 85.9536) (width 0.4064) (layer "F.Cu") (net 1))
 (segment (start 143.0147 115.5192) (end 152.1587 106.3752) (width 0.4064) (layer "F.Cu") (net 16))
 (segment (start 152.1587 97.6884) (end 152.3111 97.3836) (width 0.4064) (layer "F.Cu") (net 16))
 (segment (start 144.3863 122.8344) (end 144.6911 122.7836) (width 0.4064) (layer "F.Cu") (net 16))
 (segment (start 152.1587 106.3752) (end 152.1587 97.6884) (width 0.4064) (layer "F.Cu") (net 16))
 (segment (start 144.3863 122.8344) (end 143.0147 121.4628) (width 0.4064) (layer "F.Cu") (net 16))
 (segment (start 143.0147 121.4628) (end 143.0147 115.5192) (width 0.4064) (layer "F.Cu") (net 16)))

